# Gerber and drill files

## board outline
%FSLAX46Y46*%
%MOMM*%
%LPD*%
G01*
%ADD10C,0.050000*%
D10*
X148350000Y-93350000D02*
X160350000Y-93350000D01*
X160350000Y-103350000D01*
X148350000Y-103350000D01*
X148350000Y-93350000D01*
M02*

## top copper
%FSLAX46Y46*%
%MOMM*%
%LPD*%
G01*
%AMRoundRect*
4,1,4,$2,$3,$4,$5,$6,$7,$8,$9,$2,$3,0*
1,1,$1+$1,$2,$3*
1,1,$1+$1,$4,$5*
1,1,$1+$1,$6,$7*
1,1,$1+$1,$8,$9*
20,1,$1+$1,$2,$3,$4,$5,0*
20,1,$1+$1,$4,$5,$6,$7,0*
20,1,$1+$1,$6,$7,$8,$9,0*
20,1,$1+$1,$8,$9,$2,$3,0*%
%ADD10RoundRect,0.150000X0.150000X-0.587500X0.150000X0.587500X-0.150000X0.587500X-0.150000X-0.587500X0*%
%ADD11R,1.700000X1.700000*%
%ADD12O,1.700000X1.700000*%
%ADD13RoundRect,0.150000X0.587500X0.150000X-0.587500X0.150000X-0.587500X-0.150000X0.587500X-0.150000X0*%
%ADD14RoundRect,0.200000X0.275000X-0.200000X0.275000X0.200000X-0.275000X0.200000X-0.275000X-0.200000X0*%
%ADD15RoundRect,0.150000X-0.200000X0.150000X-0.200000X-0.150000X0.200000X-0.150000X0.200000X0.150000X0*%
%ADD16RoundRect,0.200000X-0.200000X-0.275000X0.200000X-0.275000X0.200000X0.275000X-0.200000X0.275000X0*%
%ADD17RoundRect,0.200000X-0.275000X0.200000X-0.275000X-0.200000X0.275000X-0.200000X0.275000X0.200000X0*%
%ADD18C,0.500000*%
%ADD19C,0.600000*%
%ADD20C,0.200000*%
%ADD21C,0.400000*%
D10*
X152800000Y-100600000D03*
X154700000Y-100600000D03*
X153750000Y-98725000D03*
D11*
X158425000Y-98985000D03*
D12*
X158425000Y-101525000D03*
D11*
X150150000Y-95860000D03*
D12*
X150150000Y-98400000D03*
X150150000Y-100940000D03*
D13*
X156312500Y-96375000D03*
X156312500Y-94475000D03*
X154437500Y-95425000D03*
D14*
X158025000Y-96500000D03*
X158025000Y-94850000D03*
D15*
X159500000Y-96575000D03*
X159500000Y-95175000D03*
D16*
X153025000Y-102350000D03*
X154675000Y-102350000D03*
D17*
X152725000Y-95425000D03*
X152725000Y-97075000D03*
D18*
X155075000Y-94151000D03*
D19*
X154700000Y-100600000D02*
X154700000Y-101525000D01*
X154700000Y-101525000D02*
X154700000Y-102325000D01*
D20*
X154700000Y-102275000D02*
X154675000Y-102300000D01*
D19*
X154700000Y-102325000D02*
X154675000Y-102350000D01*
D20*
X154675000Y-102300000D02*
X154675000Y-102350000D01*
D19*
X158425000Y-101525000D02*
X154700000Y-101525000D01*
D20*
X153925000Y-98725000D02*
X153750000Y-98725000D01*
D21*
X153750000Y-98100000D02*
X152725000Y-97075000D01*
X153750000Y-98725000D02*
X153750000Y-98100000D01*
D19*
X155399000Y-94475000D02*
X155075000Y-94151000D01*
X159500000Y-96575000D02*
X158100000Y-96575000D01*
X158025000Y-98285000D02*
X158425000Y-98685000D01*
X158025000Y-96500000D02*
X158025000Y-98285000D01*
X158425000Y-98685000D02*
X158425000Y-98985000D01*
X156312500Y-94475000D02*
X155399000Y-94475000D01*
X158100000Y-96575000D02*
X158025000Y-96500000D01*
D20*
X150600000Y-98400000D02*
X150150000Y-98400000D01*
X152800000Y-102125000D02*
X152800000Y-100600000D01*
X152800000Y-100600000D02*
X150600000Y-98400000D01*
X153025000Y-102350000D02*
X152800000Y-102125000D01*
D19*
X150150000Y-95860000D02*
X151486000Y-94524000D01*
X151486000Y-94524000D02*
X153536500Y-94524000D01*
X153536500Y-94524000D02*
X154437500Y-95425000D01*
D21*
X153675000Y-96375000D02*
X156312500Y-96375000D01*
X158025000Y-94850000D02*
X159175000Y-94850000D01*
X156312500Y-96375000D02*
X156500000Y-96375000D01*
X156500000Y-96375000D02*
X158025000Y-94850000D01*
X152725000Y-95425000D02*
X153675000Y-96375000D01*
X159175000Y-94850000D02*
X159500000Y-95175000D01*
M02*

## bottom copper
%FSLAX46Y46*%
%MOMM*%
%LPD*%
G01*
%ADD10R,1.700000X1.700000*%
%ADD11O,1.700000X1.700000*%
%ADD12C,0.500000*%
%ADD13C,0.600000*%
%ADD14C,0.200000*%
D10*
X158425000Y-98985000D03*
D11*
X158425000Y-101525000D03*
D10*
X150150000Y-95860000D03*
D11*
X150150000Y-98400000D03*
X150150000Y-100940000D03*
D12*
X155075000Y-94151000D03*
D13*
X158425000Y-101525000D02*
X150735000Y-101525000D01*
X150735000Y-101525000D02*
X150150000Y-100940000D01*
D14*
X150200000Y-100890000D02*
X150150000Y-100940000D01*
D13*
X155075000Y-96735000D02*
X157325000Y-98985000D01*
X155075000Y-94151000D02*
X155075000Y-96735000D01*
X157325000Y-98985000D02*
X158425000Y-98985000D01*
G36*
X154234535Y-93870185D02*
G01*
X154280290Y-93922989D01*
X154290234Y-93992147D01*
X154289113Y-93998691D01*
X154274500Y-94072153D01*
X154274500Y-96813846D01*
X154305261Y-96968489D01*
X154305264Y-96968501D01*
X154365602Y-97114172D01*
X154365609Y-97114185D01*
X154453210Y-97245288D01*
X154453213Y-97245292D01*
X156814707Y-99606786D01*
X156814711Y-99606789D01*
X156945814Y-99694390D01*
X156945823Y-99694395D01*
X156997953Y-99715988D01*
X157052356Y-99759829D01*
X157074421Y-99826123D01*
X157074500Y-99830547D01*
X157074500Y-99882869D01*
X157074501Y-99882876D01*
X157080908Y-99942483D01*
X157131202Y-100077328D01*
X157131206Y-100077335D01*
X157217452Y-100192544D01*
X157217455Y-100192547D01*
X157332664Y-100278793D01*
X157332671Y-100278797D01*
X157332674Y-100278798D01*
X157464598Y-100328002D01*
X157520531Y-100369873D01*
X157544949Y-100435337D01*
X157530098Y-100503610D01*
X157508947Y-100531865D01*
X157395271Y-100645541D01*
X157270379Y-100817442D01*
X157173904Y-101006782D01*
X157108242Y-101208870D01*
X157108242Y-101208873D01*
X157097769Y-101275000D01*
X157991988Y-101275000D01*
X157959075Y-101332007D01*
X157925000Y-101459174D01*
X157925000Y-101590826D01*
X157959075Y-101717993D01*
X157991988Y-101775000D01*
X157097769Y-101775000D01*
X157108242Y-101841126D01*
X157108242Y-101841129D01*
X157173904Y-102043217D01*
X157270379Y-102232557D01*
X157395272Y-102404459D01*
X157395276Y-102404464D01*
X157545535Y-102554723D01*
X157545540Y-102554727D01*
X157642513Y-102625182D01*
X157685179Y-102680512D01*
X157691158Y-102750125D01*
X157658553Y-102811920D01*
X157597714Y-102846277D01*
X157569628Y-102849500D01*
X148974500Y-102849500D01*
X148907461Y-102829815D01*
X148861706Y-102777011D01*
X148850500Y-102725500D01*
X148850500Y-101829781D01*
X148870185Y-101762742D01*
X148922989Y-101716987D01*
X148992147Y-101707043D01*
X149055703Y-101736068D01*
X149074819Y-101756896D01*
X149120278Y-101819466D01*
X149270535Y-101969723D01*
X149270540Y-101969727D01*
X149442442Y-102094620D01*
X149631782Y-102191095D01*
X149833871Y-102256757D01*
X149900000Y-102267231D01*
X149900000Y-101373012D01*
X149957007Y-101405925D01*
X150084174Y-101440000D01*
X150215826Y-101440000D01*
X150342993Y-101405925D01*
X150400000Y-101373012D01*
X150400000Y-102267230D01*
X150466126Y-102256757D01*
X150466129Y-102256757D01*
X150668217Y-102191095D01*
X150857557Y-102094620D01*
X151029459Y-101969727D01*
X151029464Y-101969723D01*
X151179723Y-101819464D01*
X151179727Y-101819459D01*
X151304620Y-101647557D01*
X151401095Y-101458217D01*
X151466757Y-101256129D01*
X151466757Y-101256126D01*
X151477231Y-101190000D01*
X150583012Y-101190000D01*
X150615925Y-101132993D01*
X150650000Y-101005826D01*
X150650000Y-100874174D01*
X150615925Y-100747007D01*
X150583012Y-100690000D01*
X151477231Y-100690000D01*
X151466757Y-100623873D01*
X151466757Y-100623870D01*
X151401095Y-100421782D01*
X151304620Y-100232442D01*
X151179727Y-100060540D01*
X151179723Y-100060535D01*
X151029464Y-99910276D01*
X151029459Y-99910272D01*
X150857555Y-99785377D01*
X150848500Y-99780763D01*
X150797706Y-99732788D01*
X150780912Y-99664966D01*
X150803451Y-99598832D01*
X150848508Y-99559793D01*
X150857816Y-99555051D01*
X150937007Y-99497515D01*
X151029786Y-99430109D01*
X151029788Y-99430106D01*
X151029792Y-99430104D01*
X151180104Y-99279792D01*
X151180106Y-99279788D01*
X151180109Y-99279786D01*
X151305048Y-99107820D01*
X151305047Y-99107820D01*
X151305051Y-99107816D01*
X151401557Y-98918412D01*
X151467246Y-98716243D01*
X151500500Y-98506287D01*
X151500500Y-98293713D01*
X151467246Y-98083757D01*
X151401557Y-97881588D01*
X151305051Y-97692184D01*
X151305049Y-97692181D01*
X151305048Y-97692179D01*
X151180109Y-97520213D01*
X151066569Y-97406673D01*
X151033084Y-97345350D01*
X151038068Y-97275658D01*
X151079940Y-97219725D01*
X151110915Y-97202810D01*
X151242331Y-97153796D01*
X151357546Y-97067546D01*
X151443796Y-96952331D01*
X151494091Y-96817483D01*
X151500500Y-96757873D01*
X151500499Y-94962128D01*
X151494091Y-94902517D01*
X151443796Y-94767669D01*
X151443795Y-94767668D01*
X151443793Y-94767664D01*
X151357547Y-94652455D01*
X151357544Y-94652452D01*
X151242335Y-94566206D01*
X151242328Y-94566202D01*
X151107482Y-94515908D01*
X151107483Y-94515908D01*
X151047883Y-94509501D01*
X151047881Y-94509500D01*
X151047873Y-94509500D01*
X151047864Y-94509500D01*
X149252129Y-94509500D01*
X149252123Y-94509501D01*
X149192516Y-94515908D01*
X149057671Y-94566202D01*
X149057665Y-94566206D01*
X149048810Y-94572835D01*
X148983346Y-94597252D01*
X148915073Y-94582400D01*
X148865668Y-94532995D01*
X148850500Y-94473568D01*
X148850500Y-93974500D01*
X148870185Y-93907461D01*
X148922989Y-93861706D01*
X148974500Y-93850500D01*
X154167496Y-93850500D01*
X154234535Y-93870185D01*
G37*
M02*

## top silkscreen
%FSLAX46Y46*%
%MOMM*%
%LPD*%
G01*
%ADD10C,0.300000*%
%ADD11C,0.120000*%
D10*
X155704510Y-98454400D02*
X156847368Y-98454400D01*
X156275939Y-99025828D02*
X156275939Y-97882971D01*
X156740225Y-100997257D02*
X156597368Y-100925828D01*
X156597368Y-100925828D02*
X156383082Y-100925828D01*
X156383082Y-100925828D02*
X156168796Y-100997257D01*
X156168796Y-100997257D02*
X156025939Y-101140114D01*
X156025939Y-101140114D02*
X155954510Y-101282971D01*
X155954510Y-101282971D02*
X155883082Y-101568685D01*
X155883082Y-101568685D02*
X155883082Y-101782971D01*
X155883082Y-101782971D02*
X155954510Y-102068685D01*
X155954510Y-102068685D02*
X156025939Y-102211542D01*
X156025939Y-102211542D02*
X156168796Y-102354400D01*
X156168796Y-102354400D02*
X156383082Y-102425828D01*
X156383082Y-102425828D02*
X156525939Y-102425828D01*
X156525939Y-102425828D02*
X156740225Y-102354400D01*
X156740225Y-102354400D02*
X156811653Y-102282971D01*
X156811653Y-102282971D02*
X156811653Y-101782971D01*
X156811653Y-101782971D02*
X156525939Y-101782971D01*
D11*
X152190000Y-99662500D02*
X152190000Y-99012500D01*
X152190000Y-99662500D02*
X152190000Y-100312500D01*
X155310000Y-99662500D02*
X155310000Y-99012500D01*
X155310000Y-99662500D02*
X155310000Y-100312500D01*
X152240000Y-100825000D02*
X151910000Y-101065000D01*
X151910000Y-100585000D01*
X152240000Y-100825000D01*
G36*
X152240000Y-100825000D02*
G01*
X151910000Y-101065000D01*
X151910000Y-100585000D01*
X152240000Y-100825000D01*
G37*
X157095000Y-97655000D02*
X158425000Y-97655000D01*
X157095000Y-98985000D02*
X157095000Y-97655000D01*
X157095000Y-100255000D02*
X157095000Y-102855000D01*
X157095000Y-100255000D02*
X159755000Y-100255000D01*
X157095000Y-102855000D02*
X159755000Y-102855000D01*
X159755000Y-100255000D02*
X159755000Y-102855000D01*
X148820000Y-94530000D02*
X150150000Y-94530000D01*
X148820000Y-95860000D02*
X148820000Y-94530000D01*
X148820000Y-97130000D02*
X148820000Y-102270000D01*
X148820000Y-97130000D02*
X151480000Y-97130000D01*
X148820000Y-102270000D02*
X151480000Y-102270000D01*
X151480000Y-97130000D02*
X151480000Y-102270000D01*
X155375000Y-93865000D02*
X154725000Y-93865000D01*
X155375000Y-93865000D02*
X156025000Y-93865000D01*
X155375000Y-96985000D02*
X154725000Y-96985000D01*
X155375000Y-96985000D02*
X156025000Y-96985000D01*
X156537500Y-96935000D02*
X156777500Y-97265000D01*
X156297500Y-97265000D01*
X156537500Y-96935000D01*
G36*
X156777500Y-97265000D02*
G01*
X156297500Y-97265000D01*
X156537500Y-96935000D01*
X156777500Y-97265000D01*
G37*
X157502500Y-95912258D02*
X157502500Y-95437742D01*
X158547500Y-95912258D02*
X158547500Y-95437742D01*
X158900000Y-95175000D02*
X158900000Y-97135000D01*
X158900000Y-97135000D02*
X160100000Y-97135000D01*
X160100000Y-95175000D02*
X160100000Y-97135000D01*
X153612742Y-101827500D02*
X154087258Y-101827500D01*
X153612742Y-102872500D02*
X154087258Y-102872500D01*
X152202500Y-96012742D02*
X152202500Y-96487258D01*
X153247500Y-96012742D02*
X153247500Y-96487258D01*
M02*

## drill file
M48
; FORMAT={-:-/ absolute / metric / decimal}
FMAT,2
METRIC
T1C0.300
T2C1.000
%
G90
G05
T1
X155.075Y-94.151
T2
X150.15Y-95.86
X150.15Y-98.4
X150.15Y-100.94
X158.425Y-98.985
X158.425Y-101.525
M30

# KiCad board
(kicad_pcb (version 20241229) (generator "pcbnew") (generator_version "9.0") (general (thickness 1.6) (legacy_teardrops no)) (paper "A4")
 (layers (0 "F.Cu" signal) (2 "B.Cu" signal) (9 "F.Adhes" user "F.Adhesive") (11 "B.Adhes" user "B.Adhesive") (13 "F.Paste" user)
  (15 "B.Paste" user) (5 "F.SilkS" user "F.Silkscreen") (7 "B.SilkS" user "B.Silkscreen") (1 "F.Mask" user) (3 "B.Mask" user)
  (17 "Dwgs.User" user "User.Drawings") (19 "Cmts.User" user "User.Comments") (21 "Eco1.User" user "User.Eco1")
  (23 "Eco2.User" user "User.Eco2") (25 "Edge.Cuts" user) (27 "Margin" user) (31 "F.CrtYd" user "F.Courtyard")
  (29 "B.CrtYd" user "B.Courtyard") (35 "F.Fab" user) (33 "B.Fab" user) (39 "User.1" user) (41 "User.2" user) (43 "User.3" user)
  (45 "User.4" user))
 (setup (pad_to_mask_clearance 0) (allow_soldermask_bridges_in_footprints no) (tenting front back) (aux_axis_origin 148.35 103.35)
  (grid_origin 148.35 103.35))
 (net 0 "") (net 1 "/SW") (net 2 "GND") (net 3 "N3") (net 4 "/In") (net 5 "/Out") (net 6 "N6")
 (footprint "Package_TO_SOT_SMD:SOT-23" (layer "F.Cu") (at 153.75 99.6625 90)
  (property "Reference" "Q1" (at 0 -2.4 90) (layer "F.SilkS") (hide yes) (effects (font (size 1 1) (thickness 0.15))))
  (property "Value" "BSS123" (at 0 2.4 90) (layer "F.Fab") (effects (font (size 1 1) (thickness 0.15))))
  (fp_line (start 0 -1.56) (end 0.65 -1.56) (stroke (width 0.12) (type solid)) (layer "F.SilkS"))
  (fp_line (start 0 -1.56) (end -0.65 -1.56) (stroke (width 0.12) (type solid)) (layer "F.SilkS"))
  (fp_line (start 0 1.56) (end 0.65 1.56) (stroke (width 0.12) (type solid)) (layer "F.SilkS"))
  (fp_line (start 0 1.56) (end -0.65 1.56) (stroke (width 0.12) (type solid)) (layer "F.SilkS"))
  (fp_poly
   (pts (xy -1.1625 -1.51) (xy -1.4025 -1.84) (xy -0.9225 -1.84) (xy -1.1625 -1.51)) (stroke (width 0.12) (type solid)) (fill yes)
   (layer "F.SilkS"))
  (pad "1" smd roundrect (at -0.9375 -0.95 90) (size 1.475 0.6) (layers "F.Cu" "F.Mask" "F.Paste") (roundrect_rratio 0.25) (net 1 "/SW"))
  (pad "2" smd roundrect (at -0.9375 0.95 90) (size 1.475 0.6) (layers "F.Cu" "F.Mask" "F.Paste") (roundrect_rratio 0.25) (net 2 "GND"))
  (pad "3" smd roundrect (at 0.9375 0 90) (size 1.475 0.6) (layers "F.Cu" "F.Mask" "F.Paste") (roundrect_rratio 0.25) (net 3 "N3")))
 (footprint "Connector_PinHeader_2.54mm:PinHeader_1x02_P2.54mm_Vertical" (layer "F.Cu") (at 158.425 98.985)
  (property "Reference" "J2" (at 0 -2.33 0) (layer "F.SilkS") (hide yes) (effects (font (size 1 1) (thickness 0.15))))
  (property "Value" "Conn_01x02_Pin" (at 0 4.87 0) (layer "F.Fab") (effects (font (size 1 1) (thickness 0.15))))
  (fp_line (start -1.33 -1.33) (end 0 -1.33) (stroke (width 0.12) (type solid)) (layer "F.SilkS"))
  (fp_line (start -1.33 0) (end -1.33 -1.33) (stroke (width 0.12) (type solid)) (layer "F.SilkS"))
  (fp_line (start -1.33 1.27) (end -1.33 3.87) (stroke (width 0.12) (type solid)) (layer "F.SilkS"))
  (fp_line (start -1.33 1.27) (end 1.33 1.27) (stroke (width 0.12) (type solid)) (layer "F.SilkS"))
  (fp_line (start -1.33 3.87) (end 1.33 3.87) (stroke (width 0.12) (type solid)) (layer "F.SilkS"))
  (fp_line (start 1.33 1.27) (end 1.33 3.87) (stroke (width 0.12) (type solid)) (layer "F.SilkS"))
  (pad "1" thru_hole rect (at 0 0) (size 1.7 1.7) (drill 1) (layers "*.Cu" "*.Mask") (remove_unused_layers no) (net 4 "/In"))
  (pad "2" thru_hole oval (at 0 2.54) (size 1.7 1.7) (drill 1) (layers "*.Cu" "*.Mask") (remove_unused_layers no) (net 2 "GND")))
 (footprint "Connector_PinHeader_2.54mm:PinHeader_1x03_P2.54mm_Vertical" (layer "F.Cu") (at 150.15 95.86)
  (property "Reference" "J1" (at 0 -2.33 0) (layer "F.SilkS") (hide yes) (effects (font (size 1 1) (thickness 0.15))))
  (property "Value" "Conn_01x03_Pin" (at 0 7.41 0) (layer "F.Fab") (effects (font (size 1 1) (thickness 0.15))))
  (fp_line (start -1.33 -1.33) (end 0 -1.33) (stroke (width 0.12) (type solid)) (layer "F.SilkS"))
  (fp_line (start -1.33 0) (end -1.33 -1.33) (stroke (width 0.12) (type solid)) (layer "F.SilkS"))
  (fp_line (start -1.33 1.27) (end -1.33 6.41) (stroke (width 0.12) (type solid)) (layer "F.SilkS"))
  (fp_line (start -1.33 1.27) (end 1.33 1.27) (stroke (width 0.12) (type solid)) (layer "F.SilkS"))
  (fp_line (start -1.33 6.41) (end 1.33 6.41) (stroke (width 0.12) (type solid)) (layer "F.SilkS"))
  (fp_line (start 1.33 1.27) (end 1.33 6.41) (stroke (width 0.12) (type solid)) (layer "F.SilkS"))
  (pad "1" thru_hole rect (at 0 0) (size 1.7 1.7) (drill 1) (layers "*.Cu" "*.Mask") (remove_unused_layers no) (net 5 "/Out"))
  (pad "2" thru_hole oval (at 0 2.54) (size 1.7 1.7) (drill 1) (layers "*.Cu" "*.Mask") (remove_unused_layers no) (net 1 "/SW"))
  (pad "3" thru_hole oval (at 0 5.08) (size 1.7 1.7) (drill 1) (layers "*.Cu" "*.Mask") (remove_unused_layers no) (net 2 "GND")))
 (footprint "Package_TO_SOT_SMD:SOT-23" (layer "F.Cu") (at 155.375 95.425 180)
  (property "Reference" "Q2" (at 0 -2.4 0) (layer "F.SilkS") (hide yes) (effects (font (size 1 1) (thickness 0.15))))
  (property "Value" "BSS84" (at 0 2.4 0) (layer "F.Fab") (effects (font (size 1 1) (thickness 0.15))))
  (fp_line (start 0 1.56) (end 0.65 1.56) (stroke (width 0.12) (type solid)) (layer "F.SilkS"))
  (fp_line (start 0 1.56) (end -0.65 1.56) (stroke (width 0.12) (type solid)) (layer "F.SilkS"))
  (fp_line (start 0 -1.56) (end 0.65 -1.56) (stroke (width 0.12) (type solid)) (layer "F.SilkS"))
  (fp_line (start 0 -1.56) (end -0.65 -1.56) (stroke (width 0.12) (type solid)) (layer "F.SilkS"))
  (fp_poly
   (pts (xy -1.1625 -1.51) (xy -1.4025 -1.84) (xy -0.9225 -1.84) (xy -1.1625 -1.51)) (stroke (width 0.12) (type solid)) (fill yes)
   (layer "F.SilkS"))
  (pad "1" smd roundrect (at -0.9375 -0.95 180) (size 1.475 0.6) (layers "F.Cu" "F.Mask" "F.Paste") (roundrect_rratio 0.25) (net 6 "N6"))
  (pad "2" smd roundrect (at -0.9375 0.95 180) (size 1.475 0.6) (layers "F.Cu" "F.Mask" "F.Paste") (roundrect_rratio 0.25) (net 4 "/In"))
  (pad "3" smd roundrect (at 0.9375 0 180) (size 1.475 0.6) (layers "F.Cu" "F.Mask" "F.Paste") (roundrect_rratio 0.25) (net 5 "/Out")))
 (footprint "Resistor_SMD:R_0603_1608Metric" (layer "F.Cu") (at 158.025 95.675 90)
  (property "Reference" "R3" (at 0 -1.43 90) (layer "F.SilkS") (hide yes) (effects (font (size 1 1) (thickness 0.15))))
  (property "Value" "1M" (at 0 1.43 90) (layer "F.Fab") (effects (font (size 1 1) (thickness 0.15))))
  (fp_line (start -0.237258 -0.5225) (end 0.237258 -0.5225) (stroke (width 0.12) (type solid)) (layer "F.SilkS"))
  (fp_line (start -0.237258 0.5225) (end 0.237258 0.5225) (stroke (width 0.12) (type solid)) (layer "F.SilkS"))
  (pad "1" smd roundrect (at -0.825 0 90) (size 0.8 0.95) (layers "F.Cu" "F.Mask" "F.Paste") (roundrect_rratio 0.25) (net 4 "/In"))
  (pad "2" smd roundrect (at 0.825 0 90) (size 0.8 0.95) (layers "F.Cu" "F.Mask" "F.Paste") (roundrect_rratio 0.25) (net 6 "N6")))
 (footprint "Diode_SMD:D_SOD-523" (layer "F.Cu") (at 159.5 95.875 90)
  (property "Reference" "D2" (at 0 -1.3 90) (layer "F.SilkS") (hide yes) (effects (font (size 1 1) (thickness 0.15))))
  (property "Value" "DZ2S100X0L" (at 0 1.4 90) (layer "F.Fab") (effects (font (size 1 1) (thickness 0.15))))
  (fp_line (start 0.7 -0.6) (end -1.26 -0.6) (stroke (width 0.12) (type solid)) (layer "F.SilkS"))
  (fp_line (start -1.26 -0.6) (end -1.26 0.6) (stroke (width 0.12) (type solid)) (layer "F.SilkS"))
  (fp_line (start 0.7 0.6) (end -1.26 0.6) (stroke (width 0.12) (type solid)) (layer "F.SilkS"))
  (pad "1" smd roundrect (at -0.7 0 270) (size 0.6 0.7) (layers "F.Cu" "F.Mask" "F.Paste") (roundrect_rratio 0.25) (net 4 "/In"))
  (pad "2" smd roundrect (at 0.7 0 270) (size 0.6 0.7) (layers "F.Cu" "F.Mask" "F.Paste") (roundrect_rratio 0.25) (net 6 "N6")))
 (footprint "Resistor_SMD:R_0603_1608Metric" (layer "F.Cu") (at 153.85 102.35)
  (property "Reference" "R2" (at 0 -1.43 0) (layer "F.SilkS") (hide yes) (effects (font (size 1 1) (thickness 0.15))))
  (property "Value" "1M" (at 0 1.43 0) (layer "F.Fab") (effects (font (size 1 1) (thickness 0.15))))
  (fp_line (start -0.237258 -0.5225) (end 0.237258 -0.5225) (stroke (width 0.12) (type solid)) (layer "F.SilkS"))
  (fp_line (start -0.237258 0.5225) (end 0.237258 0.5225) (stroke (width 0.12) (type solid)) (layer "F.SilkS"))
  (pad "1" smd roundrect (at -0.825 0) (size 0.8 0.95) (layers "F.Cu" "F.Mask" "F.Paste") (roundrect_rratio 0.25) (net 1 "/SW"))
  (pad "2" smd roundrect (at 0.825 0) (size 0.8 0.95) (layers "F.Cu" "F.Mask" "F.Paste") (roundrect_rratio 0.25) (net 2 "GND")))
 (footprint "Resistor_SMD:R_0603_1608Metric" (layer "F.Cu") (at 152.725 96.25 -90)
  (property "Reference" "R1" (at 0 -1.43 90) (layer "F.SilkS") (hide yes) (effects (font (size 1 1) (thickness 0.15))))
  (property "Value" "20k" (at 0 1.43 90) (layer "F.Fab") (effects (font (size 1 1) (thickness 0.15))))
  (fp_line (start -0.237258 0.5225) (end 0.237258 0.5225) (stroke (width 0.12) (type solid)) (layer "F.SilkS"))
  (fp_line (start -0.237258 -0.5225) (end 0.237258 -0.5225) (stroke (width 0.12) (type solid)) (layer "F.SilkS"))
  (pad "1" smd roundrect (at -0.825 0 270) (size 0.8 0.95) (layers "F.Cu" "F.Mask" "F.Paste") (roundrect_rratio 0.25) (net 6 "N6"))
  (pad "2" smd roundrect (at 0.825 0 270) (size 0.8 0.95) (layers "F.Cu" "F.Mask" "F.Paste") (roundrect_rratio 0.25) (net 3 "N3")))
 (gr_rect (start 148.35 93.35) (end 160.35 103.35) (stroke (width 0.05) (type solid)) (fill no) (layer "Edge.Cuts"))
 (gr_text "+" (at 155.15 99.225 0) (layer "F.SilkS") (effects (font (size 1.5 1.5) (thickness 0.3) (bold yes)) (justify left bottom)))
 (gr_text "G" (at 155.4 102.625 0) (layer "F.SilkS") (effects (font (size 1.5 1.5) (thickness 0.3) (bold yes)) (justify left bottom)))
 (segment (start 154.7 100.6) (end 154.7 101.525) (width 0.6) (layer "F.Cu") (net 2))
 (segment (start 154.7 101.525) (end 154.7 102.325) (width 0.6) (layer "F.Cu") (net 2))
 (segment (start 154.7 102.275) (end 154.675 102.3) (width 0.2) (layer "F.Cu") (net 2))
 (segment (start 154.7 102.325) (end 154.675 102.35) (width 0.6) (layer "F.Cu") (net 2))
 (segment (start 154.675 102.3) (end 154.675 102.35) (width 0.2) (layer "F.Cu") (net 2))
 (segment (start 158.425 101.525) (end 154.7 101.525) (width 0.6) (layer "F.Cu") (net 2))
 (segment (start 158.425 101.525) (end 150.735 101.525) (width 0.6) (layer "B.Cu") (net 2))
 (segment (start 150.735 101.525) (end 150.15 100.94) (width 0.6) (layer "B.Cu") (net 2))
 (segment (start 150.2 100.89) (end 150.15 100.94) (width 0.2) (layer "B.Cu") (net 2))
 (segment (start 153.925 98.725) (end 153.75 98.725) (width 0.2) (layer "F.Cu") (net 3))
 (segment (start 153.75 98.1) (end 152.725 97.075) (width 0.4) (layer "F.Cu") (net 3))
 (segment (start 153.75 98.725) (end 153.75 98.1) (width 0.4) (layer "F.Cu") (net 3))
 (segment (start 155.399 94.475) (end 155.075 94.151) (width 0.6) (layer "F.Cu") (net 4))
 (segment (start 159.5 96.575) (end 158.1 96.575) (width 0.6) (layer "F.Cu") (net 4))
 (segment (start 158.025 98.285) (end 158.425 98.685) (width 0.6) (layer "F.Cu") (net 4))
 (segment (start 158.025 96.5) (end 158.025 98.285) (width 0.6) (layer "F.Cu") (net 4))
 (segment (start 158.425 98.685) (end 158.425 98.985) (width 0.6) (layer "F.Cu") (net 4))
 (segment (start 156.3125 94.475) (end 155.399 94.475) (width 0.6) (layer "F.Cu") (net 4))
 (segment (start 158.1 96.575) (end 158.025 96.5) (width 0.6) (layer "F.Cu") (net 4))
 (via (at 155.075 94.151) (size 0.5) (drill 0.3) (layers "F.Cu" "B.Cu") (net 4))
 (segment (start 155.075 96.735) (end 157.325 98.985) (width 0.6) (layer "B.Cu") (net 4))
 (segment (start 155.075 94.151) (end 155.075 96.735) (width 0.6) (layer "B.Cu") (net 4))
 (segment (start 157.325 98.985) (end 158.425 98.985) (width 0.6) (layer "B.Cu") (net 4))
 (segment (start 150.6 98.4) (end 150.15 98.4) (width 0.2) (layer "F.Cu") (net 1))
 (segment (start 152.8 102.125) (end 152.8 100.6) (width 0.2) (layer "F.Cu") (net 1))
 (segment (start 152.8 100.6) (end 150.6 98.4) (width 0.2) (layer "F.Cu") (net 1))
 (segment (start 153.025 102.35) (end 152.8 102.125) (width 0.2) (layer "F.Cu") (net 1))
 (segment (start 150.15 95.86) (end 151.486 94.524) (width 0.6) (layer "F.Cu") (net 5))
 (segment (start 151.486 94.524) (end 153.5365 94.524) (width 0.6) (layer "F.Cu") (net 5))
 (segment (start 153.5365 94.524) (end 154.4375 95.425) (width 0.6) (layer "F.Cu") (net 5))
 (segment (start 153.675 96.375) (end 156.3125 96.375) (width 0.4) (layer "F.Cu") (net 6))
 (segment (start 158.025 94.85) (end 159.175 94.85) (width 0.4) (layer "F.Cu") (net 6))
 (segment (start 156.3125 96.375) (end 156.5 96.375) (width 0.4) (layer "F.Cu") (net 6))
 (segment (start 156.5 96.375) (end 158.025 94.85) (width 0.4) (layer "F.Cu") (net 6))
 (segment (start 152.725 95.425) (end 153.675 96.375) (width 0.4) (layer "F.Cu") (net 6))
 (segment (start 159.175 94.85) (end 159.5 95.175) (width 0.4) (layer "F.Cu") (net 6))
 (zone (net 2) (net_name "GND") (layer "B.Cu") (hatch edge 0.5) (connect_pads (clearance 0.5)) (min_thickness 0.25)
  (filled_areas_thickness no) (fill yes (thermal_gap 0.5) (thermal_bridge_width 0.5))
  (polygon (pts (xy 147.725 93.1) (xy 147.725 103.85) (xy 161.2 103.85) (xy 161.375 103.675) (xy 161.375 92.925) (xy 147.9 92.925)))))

